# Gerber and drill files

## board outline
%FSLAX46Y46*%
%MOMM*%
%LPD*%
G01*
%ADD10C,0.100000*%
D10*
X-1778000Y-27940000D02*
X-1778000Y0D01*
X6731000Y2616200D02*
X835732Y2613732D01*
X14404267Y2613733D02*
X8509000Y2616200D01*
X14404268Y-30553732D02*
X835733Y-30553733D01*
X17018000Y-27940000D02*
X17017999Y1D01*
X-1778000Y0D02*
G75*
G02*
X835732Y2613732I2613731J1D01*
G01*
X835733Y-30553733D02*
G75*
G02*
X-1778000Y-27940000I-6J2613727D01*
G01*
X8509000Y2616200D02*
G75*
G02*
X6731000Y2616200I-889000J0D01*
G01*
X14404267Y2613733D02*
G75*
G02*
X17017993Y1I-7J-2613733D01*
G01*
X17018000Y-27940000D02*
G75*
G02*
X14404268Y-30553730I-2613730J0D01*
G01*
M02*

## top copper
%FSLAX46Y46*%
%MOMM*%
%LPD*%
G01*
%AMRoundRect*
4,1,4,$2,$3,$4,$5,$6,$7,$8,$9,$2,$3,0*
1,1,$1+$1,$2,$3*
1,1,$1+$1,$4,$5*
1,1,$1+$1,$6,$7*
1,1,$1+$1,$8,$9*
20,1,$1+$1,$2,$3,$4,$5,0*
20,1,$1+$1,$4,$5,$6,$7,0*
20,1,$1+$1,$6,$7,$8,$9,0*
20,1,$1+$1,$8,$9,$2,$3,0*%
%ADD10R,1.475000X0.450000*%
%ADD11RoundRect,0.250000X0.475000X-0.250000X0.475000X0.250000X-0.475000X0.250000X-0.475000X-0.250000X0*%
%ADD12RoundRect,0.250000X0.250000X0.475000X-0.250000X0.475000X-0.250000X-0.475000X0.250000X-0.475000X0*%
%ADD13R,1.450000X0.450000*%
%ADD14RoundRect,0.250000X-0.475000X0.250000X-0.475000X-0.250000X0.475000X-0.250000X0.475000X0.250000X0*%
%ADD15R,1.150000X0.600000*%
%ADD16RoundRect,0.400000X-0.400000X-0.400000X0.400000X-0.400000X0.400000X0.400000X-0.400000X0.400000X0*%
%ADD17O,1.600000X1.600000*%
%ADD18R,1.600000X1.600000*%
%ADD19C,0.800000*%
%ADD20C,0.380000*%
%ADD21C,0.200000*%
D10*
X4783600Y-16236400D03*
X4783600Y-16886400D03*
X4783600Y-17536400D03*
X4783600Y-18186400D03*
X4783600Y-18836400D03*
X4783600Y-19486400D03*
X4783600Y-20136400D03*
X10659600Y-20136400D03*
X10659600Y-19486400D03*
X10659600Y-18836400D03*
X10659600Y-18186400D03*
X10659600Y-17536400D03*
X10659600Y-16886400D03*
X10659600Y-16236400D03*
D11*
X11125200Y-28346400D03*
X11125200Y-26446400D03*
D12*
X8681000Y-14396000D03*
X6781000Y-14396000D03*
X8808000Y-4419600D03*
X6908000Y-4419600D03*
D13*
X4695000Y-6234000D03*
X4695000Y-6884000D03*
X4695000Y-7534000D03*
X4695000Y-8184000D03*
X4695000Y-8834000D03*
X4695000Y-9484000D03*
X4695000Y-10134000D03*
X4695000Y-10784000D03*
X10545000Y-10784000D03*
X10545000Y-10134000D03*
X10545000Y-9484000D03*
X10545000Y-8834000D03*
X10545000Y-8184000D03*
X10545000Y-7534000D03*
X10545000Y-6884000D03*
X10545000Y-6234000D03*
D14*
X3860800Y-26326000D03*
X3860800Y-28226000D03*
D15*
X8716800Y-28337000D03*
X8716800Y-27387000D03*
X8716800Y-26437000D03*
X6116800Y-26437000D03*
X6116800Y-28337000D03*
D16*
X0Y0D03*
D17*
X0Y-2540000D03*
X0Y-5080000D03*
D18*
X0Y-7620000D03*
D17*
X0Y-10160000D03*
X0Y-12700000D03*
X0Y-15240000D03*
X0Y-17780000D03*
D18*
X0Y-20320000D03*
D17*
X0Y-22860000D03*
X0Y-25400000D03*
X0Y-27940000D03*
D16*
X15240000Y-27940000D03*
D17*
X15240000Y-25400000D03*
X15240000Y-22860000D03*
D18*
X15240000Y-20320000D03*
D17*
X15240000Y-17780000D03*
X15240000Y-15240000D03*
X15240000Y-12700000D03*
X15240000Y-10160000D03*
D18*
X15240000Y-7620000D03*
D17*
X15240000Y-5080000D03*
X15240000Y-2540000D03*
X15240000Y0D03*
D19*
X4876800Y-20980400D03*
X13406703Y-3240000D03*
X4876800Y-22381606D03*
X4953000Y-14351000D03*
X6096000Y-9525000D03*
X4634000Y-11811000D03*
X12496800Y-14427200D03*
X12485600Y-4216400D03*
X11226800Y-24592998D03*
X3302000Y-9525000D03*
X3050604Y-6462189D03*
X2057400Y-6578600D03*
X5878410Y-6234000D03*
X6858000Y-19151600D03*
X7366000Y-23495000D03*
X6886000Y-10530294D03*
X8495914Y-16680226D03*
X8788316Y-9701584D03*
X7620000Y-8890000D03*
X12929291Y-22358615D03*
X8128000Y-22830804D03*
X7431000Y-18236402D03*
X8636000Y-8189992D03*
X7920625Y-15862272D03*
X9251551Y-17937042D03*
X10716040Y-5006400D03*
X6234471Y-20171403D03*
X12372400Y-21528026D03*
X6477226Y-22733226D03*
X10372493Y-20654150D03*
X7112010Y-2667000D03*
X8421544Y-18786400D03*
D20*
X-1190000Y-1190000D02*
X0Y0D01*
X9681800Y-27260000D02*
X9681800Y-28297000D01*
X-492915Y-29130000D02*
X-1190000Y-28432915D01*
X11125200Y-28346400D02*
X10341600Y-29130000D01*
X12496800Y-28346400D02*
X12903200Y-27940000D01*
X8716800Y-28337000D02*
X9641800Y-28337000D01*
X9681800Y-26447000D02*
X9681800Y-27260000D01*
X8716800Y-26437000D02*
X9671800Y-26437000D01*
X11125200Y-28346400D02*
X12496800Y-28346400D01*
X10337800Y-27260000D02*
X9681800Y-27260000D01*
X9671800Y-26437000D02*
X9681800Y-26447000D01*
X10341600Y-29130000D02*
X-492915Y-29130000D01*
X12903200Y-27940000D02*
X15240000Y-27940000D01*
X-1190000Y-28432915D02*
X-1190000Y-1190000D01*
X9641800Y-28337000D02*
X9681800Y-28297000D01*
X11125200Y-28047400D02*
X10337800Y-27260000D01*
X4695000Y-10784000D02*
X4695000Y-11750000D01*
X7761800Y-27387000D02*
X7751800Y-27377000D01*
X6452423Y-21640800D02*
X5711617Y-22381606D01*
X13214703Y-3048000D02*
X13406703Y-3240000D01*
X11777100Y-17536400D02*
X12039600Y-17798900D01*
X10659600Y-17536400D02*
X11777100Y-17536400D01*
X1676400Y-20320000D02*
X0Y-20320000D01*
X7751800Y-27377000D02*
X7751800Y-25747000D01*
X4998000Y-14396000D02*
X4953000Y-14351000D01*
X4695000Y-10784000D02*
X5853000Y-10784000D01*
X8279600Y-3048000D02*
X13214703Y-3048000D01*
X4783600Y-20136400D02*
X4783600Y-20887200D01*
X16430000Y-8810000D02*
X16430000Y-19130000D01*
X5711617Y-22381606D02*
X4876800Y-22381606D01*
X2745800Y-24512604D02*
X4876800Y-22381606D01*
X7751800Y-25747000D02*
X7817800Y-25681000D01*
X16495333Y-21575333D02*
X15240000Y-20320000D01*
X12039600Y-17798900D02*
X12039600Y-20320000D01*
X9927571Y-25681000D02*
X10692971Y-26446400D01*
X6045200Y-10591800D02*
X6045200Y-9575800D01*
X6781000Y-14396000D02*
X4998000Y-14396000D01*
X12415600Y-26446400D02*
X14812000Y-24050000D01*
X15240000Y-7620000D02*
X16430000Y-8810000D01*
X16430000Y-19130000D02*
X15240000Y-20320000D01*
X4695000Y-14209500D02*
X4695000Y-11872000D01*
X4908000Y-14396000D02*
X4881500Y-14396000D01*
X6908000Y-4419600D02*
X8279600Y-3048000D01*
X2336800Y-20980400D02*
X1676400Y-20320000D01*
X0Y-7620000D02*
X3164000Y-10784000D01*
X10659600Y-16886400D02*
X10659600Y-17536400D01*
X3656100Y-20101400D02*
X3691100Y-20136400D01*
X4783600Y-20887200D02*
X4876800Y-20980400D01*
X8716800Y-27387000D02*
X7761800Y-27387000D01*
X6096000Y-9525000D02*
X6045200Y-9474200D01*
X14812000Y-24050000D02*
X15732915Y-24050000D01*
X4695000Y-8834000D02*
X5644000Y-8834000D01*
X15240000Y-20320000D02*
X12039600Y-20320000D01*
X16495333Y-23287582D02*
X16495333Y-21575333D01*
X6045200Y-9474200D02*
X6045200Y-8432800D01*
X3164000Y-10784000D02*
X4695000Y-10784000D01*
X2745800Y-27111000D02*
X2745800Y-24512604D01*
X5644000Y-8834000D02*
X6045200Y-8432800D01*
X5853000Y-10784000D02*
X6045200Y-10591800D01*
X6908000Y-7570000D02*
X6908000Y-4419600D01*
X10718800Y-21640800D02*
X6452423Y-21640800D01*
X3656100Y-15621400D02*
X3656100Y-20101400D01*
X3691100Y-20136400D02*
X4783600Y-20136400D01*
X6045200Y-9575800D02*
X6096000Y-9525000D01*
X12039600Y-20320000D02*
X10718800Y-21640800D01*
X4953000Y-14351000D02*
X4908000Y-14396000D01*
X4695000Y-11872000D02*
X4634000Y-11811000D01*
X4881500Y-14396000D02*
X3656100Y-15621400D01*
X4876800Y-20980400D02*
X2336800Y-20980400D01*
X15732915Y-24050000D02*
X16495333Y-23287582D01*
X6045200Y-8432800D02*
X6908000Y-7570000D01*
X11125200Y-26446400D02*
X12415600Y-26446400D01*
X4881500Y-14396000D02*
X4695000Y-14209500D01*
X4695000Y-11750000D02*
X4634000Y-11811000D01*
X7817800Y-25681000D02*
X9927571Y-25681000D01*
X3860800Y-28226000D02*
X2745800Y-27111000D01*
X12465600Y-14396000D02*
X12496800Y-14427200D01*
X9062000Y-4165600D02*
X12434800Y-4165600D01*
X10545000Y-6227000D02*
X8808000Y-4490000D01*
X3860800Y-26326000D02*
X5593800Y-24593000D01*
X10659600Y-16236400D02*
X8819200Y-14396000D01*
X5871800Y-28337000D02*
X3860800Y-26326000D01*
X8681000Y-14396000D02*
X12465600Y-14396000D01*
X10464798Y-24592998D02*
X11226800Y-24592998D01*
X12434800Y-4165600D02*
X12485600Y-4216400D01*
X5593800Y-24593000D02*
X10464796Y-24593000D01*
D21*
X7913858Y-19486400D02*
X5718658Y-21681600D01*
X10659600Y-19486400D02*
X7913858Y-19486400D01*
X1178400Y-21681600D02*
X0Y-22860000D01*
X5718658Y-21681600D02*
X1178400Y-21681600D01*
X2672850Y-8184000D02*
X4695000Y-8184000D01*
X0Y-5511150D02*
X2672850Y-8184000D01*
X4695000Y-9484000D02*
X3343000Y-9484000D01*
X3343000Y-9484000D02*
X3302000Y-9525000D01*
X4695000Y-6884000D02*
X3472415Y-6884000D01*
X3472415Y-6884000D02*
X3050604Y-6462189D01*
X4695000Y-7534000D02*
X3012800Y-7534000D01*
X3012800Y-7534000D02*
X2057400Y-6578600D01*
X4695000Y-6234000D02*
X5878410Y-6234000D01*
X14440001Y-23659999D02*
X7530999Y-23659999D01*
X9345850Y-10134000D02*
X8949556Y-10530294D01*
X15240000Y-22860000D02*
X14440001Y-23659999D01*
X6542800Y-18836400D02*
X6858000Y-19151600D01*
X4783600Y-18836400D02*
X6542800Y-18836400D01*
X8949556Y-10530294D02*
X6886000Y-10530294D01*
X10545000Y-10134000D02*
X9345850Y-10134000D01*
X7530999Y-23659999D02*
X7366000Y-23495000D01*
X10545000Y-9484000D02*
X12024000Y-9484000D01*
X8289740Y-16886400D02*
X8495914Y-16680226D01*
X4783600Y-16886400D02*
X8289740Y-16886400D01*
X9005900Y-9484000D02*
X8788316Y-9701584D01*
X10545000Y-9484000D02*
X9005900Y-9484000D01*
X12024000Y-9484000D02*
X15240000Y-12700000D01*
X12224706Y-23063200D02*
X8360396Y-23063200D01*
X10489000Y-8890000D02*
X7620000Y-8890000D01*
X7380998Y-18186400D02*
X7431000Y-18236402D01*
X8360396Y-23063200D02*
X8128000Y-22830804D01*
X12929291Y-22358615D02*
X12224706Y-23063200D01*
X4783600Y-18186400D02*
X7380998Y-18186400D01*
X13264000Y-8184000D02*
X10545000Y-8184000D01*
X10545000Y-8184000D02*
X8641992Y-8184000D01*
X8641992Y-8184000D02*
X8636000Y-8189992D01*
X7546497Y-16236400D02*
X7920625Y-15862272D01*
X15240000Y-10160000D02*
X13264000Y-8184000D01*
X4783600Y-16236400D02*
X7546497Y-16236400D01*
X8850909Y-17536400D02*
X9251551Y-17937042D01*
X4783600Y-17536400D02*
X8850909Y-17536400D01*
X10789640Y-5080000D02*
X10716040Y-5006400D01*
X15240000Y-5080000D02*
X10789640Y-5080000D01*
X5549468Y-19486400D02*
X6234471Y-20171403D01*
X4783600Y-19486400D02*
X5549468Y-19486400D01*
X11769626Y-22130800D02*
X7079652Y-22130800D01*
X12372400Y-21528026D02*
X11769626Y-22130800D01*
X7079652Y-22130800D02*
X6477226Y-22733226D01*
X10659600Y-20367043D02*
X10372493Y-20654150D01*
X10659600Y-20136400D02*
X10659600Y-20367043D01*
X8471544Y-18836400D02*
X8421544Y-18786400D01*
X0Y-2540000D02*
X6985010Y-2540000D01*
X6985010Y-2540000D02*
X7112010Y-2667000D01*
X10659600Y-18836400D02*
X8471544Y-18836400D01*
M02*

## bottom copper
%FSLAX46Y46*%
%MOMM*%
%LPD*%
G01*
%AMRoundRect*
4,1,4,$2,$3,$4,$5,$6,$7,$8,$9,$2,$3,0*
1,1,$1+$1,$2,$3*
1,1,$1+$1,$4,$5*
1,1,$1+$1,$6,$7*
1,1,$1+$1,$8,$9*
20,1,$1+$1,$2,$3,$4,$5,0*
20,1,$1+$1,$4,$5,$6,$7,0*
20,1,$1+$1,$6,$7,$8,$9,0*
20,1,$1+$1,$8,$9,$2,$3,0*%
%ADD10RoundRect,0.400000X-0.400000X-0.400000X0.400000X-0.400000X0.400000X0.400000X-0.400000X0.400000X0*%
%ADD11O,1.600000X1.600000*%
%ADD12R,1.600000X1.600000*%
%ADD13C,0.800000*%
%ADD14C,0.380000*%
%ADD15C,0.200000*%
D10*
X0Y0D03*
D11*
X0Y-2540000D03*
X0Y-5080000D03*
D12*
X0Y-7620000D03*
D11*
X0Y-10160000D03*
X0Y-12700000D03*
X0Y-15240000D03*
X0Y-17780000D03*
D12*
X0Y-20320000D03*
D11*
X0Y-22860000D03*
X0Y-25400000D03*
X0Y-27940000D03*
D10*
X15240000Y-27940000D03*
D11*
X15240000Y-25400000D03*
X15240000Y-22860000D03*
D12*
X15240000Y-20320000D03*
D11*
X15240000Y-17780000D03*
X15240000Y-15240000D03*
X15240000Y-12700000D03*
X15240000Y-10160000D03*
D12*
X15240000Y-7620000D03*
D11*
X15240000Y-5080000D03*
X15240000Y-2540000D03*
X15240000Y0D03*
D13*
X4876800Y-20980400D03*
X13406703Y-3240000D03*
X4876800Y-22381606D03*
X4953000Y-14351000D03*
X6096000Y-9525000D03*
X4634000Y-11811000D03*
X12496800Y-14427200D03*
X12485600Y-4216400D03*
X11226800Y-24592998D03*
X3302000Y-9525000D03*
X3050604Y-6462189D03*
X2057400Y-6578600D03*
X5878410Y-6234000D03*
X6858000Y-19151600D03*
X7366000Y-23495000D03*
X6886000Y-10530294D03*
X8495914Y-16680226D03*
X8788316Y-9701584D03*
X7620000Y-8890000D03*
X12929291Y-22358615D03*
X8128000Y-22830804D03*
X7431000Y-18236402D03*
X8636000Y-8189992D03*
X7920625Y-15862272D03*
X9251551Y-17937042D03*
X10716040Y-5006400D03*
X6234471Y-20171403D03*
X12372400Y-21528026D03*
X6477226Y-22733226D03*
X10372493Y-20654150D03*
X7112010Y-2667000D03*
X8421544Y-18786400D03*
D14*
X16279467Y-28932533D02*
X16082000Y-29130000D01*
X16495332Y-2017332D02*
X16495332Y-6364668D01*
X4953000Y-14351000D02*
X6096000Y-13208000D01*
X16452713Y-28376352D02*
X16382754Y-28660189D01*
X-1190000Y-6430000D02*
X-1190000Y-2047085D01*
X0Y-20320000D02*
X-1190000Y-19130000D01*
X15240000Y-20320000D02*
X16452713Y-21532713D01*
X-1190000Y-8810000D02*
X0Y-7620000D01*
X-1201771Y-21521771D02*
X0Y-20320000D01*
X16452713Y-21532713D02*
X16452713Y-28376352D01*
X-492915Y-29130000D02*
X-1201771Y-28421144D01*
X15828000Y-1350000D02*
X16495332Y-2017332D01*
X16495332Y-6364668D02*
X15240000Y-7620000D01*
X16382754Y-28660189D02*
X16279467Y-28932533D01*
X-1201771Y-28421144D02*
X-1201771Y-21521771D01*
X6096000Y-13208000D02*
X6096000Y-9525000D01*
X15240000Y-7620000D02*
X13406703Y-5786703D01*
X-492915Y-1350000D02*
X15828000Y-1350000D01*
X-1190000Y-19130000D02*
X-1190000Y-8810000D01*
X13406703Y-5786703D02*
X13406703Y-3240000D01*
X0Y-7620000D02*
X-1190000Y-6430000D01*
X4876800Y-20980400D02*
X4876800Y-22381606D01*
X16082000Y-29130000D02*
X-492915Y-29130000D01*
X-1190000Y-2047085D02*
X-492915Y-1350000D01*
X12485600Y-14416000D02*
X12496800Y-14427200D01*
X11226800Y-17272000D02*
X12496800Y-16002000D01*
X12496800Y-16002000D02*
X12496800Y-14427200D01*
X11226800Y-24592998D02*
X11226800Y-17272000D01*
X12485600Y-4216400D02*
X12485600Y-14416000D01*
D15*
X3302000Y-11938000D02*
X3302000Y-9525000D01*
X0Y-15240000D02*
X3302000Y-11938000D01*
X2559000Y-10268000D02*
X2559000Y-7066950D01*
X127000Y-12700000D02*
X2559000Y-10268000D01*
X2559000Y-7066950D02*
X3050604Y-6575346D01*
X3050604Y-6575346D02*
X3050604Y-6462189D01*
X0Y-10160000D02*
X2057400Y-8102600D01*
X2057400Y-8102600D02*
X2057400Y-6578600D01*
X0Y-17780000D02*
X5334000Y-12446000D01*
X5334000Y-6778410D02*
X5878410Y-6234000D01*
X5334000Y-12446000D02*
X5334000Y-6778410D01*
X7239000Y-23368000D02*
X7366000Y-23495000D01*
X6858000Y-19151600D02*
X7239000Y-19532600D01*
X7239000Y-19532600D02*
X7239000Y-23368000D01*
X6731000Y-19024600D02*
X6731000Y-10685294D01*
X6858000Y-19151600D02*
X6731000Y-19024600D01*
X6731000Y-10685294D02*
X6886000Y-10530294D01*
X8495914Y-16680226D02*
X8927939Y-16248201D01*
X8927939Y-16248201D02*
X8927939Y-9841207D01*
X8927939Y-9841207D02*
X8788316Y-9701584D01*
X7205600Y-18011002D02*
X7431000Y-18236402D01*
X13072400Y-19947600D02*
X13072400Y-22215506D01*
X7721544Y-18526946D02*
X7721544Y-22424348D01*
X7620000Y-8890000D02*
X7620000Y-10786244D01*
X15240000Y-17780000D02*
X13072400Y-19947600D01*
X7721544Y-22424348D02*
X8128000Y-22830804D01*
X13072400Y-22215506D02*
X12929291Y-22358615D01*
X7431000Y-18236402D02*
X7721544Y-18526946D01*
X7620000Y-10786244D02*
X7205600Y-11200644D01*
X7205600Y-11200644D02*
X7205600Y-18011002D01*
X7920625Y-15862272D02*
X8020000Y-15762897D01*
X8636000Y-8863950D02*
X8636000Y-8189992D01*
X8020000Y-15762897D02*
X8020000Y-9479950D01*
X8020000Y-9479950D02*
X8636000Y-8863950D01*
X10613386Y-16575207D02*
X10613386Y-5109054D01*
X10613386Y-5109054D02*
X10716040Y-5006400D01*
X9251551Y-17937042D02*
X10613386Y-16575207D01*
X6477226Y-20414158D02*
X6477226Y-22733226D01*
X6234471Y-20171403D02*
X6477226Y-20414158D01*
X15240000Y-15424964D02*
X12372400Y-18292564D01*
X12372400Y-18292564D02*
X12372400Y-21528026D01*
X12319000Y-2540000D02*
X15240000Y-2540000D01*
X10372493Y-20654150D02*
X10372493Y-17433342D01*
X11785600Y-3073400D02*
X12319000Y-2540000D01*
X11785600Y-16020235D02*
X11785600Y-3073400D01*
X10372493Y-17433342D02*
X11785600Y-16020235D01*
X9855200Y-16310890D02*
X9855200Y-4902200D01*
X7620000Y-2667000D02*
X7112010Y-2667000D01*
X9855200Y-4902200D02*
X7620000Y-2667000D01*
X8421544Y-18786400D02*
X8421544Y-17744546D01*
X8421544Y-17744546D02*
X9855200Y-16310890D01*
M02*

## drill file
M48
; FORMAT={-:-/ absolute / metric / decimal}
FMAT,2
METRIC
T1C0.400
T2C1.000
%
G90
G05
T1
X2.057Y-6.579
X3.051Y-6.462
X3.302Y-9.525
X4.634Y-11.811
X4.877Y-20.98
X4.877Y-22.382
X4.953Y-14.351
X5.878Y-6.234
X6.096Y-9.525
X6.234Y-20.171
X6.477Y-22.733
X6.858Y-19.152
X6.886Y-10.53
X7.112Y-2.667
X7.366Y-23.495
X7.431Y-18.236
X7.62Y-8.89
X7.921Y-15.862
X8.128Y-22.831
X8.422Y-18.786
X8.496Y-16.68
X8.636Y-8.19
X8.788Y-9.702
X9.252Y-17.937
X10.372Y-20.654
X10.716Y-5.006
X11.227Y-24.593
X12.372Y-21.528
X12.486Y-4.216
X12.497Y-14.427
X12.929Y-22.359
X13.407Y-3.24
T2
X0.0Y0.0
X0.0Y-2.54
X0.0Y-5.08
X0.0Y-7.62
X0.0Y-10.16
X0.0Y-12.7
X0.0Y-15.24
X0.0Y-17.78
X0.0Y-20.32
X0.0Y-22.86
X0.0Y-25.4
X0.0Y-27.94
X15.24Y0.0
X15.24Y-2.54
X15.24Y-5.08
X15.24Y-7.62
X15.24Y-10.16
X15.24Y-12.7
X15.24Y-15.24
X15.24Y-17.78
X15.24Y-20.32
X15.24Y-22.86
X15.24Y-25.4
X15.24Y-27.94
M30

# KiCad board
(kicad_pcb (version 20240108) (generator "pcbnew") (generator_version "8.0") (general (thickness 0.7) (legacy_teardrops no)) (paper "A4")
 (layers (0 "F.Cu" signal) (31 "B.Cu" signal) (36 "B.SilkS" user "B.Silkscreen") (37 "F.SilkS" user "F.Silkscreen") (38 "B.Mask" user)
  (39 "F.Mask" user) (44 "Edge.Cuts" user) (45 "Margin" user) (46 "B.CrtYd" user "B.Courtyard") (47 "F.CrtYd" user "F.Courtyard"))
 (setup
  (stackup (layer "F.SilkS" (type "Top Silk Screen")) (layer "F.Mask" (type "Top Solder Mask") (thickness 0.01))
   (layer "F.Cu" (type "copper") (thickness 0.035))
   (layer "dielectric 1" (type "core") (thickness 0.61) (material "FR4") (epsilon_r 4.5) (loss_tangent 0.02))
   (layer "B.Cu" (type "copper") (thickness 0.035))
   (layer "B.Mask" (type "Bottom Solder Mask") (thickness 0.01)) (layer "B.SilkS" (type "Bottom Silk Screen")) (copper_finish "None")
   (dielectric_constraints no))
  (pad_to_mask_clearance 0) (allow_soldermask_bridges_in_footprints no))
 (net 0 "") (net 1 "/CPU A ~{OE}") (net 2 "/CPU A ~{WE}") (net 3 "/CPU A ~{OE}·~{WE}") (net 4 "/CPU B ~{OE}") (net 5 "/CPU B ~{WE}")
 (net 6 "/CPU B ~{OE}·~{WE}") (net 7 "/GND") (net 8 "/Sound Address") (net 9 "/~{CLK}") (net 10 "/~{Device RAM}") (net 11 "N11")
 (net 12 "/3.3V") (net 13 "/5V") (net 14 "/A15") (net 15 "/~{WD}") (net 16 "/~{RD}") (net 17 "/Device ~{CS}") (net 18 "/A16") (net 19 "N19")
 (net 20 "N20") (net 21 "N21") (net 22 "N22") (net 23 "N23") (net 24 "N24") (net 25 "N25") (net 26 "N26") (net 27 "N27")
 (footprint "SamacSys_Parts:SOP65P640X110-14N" (layer "F.Cu") (at 7.7216 18.1864)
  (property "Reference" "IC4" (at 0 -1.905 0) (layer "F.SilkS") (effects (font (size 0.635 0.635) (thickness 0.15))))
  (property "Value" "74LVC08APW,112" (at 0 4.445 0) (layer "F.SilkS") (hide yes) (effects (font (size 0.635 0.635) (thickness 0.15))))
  (pad "1" smd rect (at -2.938 -1.95 90) (size 0.45 1.475) (layers "F.Cu" "F.Paste" "F.Mask") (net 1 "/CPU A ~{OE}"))
  (pad "2" smd rect (at -2.938 -1.3 90) (size 0.45 1.475) (layers "F.Cu" "F.Paste" "F.Mask") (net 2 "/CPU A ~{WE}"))
  (pad "3" smd rect (at -2.938 -0.65 90) (size 0.45 1.475) (layers "F.Cu" "F.Paste" "F.Mask") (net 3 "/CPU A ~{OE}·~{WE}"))
  (pad "4" smd rect (at -2.938 0 90) (size 0.45 1.475) (layers "F.Cu" "F.Paste" "F.Mask") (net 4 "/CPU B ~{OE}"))
  (pad "5" smd rect (at -2.938 0.65 90) (size 0.45 1.475) (layers "F.Cu" "F.Paste" "F.Mask") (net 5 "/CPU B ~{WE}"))
  (pad "6" smd rect (at -2.938 1.3 90) (size 0.45 1.475) (layers "F.Cu" "F.Paste" "F.Mask") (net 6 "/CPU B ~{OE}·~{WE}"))
  (pad "7" smd rect (at -2.938 1.95 90) (size 0.45 1.475) (layers "F.Cu" "F.Paste" "F.Mask") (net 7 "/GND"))
  (pad "8" smd rect (at 2.938 1.95 90) (size 0.45 1.475) (layers "F.Cu" "F.Paste" "F.Mask") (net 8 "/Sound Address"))
  (pad "9" smd rect (at 2.938 1.3 90) (size 0.45 1.475) (layers "F.Cu" "F.Paste" "F.Mask") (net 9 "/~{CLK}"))
  (pad "10" smd rect (at 2.938 0.65 90) (size 0.45 1.475) (layers "F.Cu" "F.Paste" "F.Mask") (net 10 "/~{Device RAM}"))
  (pad "11" smd rect (at 2.938 0 90) (size 0.45 1.475) (layers "F.Cu" "F.Paste" "F.Mask") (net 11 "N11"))
  (pad "12" smd rect (at 2.938 -0.65 90) (size 0.45 1.475) (layers "F.Cu" "F.Paste" "F.Mask") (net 7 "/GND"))
  (pad "13" smd rect (at 2.938 -1.3 90) (size 0.45 1.475) (layers "F.Cu" "F.Paste" "F.Mask") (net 7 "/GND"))
  (pad "14" smd rect (at 2.938 -1.95 90) (size 0.45 1.475) (layers "F.Cu" "F.Paste" "F.Mask") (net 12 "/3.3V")))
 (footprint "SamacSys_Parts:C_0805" (layer "F.Cu") (at 11.1252 27.4124)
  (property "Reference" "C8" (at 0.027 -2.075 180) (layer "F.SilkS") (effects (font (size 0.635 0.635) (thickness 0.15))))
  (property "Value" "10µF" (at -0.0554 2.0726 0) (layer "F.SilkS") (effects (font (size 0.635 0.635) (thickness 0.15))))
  (pad "1" smd roundrect (at 0 0.934 90) (size 1 1.45) (layers "F.Cu" "F.Paste" "F.Mask") (roundrect_rratio 0.25) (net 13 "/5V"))
  (pad "2" smd roundrect (at 0 -0.966 90) (size 1 1.45) (layers "F.Cu" "F.Paste" "F.Mask") (roundrect_rratio 0.25) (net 7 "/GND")))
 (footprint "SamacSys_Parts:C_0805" (layer "F.Cu") (at 7.747 14.396 90)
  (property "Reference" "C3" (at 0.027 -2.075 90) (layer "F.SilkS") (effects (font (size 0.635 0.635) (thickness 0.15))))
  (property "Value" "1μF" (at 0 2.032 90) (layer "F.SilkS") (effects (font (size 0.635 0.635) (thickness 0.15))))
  (pad "1" smd roundrect (at 0 0.934 180) (size 1 1.45) (layers "F.Cu" "F.Paste" "F.Mask") (roundrect_rratio 0.25) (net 12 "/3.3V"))
  (pad "2" smd roundrect (at 0 -0.966 180) (size 1 1.45) (layers "F.Cu" "F.Paste" "F.Mask") (roundrect_rratio 0.25) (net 7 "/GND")))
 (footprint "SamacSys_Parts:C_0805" (layer "F.Cu") (at 7.874 4.4196 90)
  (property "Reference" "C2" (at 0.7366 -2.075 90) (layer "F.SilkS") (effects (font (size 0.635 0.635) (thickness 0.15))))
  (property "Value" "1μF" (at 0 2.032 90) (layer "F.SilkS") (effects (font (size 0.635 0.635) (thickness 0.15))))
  (pad "1" smd roundrect (at 0 0.934 180) (size 1 1.45) (layers "F.Cu" "F.Paste" "F.Mask") (roundrect_rratio 0.25) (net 12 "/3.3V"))
  (pad "2" smd roundrect (at 0 -0.966 180) (size 1 1.45) (layers "F.Cu" "F.Paste" "F.Mask") (roundrect_rratio 0.25) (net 7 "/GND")))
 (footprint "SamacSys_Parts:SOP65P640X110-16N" (layer "F.Cu") (at 7.62 8.509)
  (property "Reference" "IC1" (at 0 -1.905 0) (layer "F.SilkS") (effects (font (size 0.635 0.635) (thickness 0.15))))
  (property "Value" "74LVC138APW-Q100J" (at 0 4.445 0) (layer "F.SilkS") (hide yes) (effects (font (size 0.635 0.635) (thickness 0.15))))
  (pad "1" smd rect (at -2.925 -2.275 90) (size 0.45 1.45) (layers "F.Cu" "F.Paste" "F.Mask") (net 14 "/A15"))
  (pad "2" smd rect (at -2.925 -1.625 90) (size 0.45 1.45) (layers "F.Cu" "F.Paste" "F.Mask") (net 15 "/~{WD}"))
  (pad "3" smd rect (at -2.925 -0.975 90) (size 0.45 1.45) (layers "F.Cu" "F.Paste" "F.Mask") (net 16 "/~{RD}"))
  (pad "4" smd rect (at -2.925 -0.325 90) (size 0.45 1.45) (layers "F.Cu" "F.Paste" "F.Mask") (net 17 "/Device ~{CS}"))
  (pad "5" smd rect (at -2.925 0.325 90) (size 0.45 1.45) (layers "F.Cu" "F.Paste" "F.Mask") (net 7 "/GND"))
  (pad "6" smd rect (at -2.925 0.975 90) (size 0.45 1.45) (layers "F.Cu" "F.Paste" "F.Mask") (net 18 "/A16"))
  (pad "7" smd rect (at -2.925 1.625 90) (size 0.45 1.45) (layers "F.Cu" "F.Paste" "F.Mask") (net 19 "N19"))
  (pad "8" smd rect (at -2.925 2.275 90) (size 0.45 1.45) (layers "F.Cu" "F.Paste" "F.Mask") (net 7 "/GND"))
  (pad "9" smd rect (at 2.925 2.275 90) (size 0.45 1.45) (layers "F.Cu" "F.Paste" "F.Mask") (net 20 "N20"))
  (pad "10" smd rect (at 2.925 1.625 90) (size 0.45 1.45) (layers "F.Cu" "F.Paste" "F.Mask") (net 5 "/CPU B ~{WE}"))
  (pad "11" smd rect (at 2.925 0.975 90) (size 0.45 1.45) (layers "F.Cu" "F.Paste" "F.Mask") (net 2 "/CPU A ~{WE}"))
  (pad "12" smd rect (at 2.925 0.325 90) (size 0.45 1.45) (layers "F.Cu" "F.Paste" "F.Mask") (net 4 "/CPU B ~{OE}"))
  (pad "13" smd rect (at 2.925 -0.325 90) (size 0.45 1.45) (layers "F.Cu" "F.Paste" "F.Mask") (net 1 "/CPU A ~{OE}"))
  (pad "14" smd rect (at 2.925 -0.975 90) (size 0.45 1.45) (layers "F.Cu" "F.Paste" "F.Mask") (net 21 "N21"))
  (pad "15" smd rect (at 2.925 -1.625 90) (size 0.45 1.45) (layers "F.Cu" "F.Paste" "F.Mask") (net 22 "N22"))
  (pad "16" smd rect (at 2.925 -2.275 90) (size 0.45 1.45) (layers "F.Cu" "F.Paste" "F.Mask") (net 12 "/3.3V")))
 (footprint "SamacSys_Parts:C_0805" (layer "F.Cu") (at 3.8608 27.26 180)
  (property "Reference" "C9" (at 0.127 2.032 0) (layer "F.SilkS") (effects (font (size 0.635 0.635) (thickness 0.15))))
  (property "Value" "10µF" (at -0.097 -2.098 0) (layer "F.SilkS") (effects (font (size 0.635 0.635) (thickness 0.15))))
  (pad "1" smd roundrect (at 0 0.934 270) (size 1 1.45) (layers "F.Cu" "F.Paste" "F.Mask") (roundrect_rratio 0.25) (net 12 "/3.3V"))
  (pad "2" smd roundrect (at 0 -0.966 270) (size 1 1.45) (layers "F.Cu" "F.Paste" "F.Mask") (roundrect_rratio 0.25) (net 7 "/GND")))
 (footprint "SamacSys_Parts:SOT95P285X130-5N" (layer "F.Cu") (at 7.4168 27.387 180)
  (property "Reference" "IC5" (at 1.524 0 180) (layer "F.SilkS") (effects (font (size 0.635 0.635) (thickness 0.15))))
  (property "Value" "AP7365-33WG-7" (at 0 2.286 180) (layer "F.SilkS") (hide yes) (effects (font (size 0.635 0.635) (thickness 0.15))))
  (pad "1" smd rect (at -1.3 -0.95 270) (size 0.6 1.15) (layers "F.Cu" "F.Paste" "F.Mask") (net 13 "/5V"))
  (pad "2" smd rect (at -1.3 0 270) (size 0.6 1.15) (layers "F.Cu" "F.Paste" "F.Mask") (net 7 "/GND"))
  (pad "3" smd rect (at -1.3 0.95 270) (size 0.6 1.15) (layers "F.Cu" "F.Paste" "F.Mask") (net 13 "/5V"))
  (pad "4" smd rect (at 1.3 0.95 270) (size 0.6 1.15) (layers "F.Cu" "F.Paste" "F.Mask") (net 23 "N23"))
  (pad "5" smd rect (at 1.3 -0.95 270) (size 0.6 1.15) (layers "F.Cu" "F.Paste" "F.Mask") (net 12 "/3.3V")))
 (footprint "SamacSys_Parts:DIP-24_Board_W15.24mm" (layer "F.Cu") (at 0 0)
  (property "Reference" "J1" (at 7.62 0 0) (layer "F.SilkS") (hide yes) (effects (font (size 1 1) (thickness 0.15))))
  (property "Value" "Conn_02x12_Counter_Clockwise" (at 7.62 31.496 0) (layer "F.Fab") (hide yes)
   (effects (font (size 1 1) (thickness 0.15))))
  (fp_line (start -1.778 27.94) (end -1.778 0) (stroke (width 0.1) (type solid)) (layer "Edge.Cuts"))
  (fp_line (start 6.731 -2.6162) (end 0.835732 -2.613732) (stroke (width 0.1) (type solid)) (layer "Edge.Cuts"))
  (fp_line (start 14.404267 -2.613733) (end 8.509 -2.6162) (stroke (width 0.1) (type solid)) (layer "Edge.Cuts"))
  (fp_line (start 14.404268 30.553732) (end 0.835733 30.553733) (stroke (width 0.1) (type solid)) (layer "Edge.Cuts"))
  (fp_line (start 17.018 27.94) (end 17.017999 -0.000001) (stroke (width 0.1) (type solid)) (layer "Edge.Cuts"))
  (fp_arc (start -1.778 0) (mid -1.012456 -1.848188) (end 0.835732 -2.613732) (stroke (width 0.1) (type solid)) (layer "Edge.Cuts"))
  (fp_arc (start 0.835733 30.553733) (mid -1.012457 29.78819) (end -1.778 27.94) (stroke (width 0.1) (type solid)) (layer "Edge.Cuts"))
  (fp_arc (start 8.509 -2.6162) (mid 7.62 -1.7272) (end 6.731 -2.6162) (stroke (width 0.1) (type default)) (layer "Edge.Cuts"))
  (fp_arc (start 14.404267 -2.613733) (mid 16.252453 -1.848189) (end 17.017999 -0.000001) (stroke (width 0.1) (type solid))
   (layer "Edge.Cuts"))
  (fp_arc (start 17.018 27.94) (mid 16.252456 29.788187) (end 14.404268 30.553732) (stroke (width 0.1) (type solid)) (layer "Edge.Cuts"))
  (pad "1" thru_hole roundrect (at 0 0) (size 1.6 1.6) (drill 1) (layers "*.Cu" "*.Mask") (remove_unused_layers no) (roundrect_rratio 0.25)
   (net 13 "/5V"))
  (pad "2" thru_hole oval (at 0 2.54) (size 1.6 1.6) (drill 1) (layers "*.Cu" "*.Mask") (remove_unused_layers no) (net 10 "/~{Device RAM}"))
  (pad "3" thru_hole oval (at 0 5.08) (size 1.6 1.6) (drill 1) (layers "*.Cu" "*.Mask") (remove_unused_layers no) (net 17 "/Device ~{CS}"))
  (pad "4" thru_hole rect (at 0 7.62) (size 1.6 1.6) (drill 1) (layers "*.Cu" "*.Mask") (remove_unused_layers no) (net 7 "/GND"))
  (pad "5" thru_hole oval (at 0 10.16) (size 1.6 1.6) (drill 1) (layers "*.Cu" "*.Mask") (remove_unused_layers no) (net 16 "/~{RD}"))
  (pad "6" thru_hole oval (at 0 12.7) (size 1.6 1.6) (drill 1) (layers "*.Cu" "*.Mask") (remove_unused_layers no) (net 15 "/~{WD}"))
  (pad "7" thru_hole oval (at 0 15.24) (size 1.6 1.6) (drill 1) (layers "*.Cu" "*.Mask") (remove_unused_layers no) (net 18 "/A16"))
  (pad "8" thru_hole oval (at 0 17.78) (size 1.6 1.6) (drill 1) (layers "*.Cu" "*.Mask") (remove_unused_layers no) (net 14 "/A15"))
  (pad "9" thru_hole rect (at 0 20.32) (size 1.6 1.6) (drill 1) (layers "*.Cu" "*.Mask") (remove_unused_layers no) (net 7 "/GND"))
  (pad "10" thru_hole oval (at 0 22.86) (size 1.6 1.6) (drill 1) (layers "*.Cu" "*.Mask") (remove_unused_layers no) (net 9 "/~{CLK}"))
  (pad "11" thru_hole oval (at 0 25.4) (size 1.6 1.6) (drill 1) (layers "*.Cu" "*.Mask") (remove_unused_layers no) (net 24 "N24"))
  (pad "12" thru_hole oval (at 0 27.94) (size 1.6 1.6) (drill 1) (layers "*.Cu" "*.Mask") (remove_unused_layers no) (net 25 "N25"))
  (pad "13" thru_hole roundrect (at 15.24 27.94) (size 1.6 1.6) (drill 1) (layers "*.Cu" "*.Mask") (remove_unused_layers no)
   (roundrect_rratio 0.25) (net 13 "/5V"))
  (pad "14" thru_hole oval (at 15.24 25.4) (size 1.6 1.6) (drill 1) (layers "*.Cu" "*.Mask") (remove_unused_layers no) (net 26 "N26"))
  (pad "15" thru_hole oval (at 15.24 22.86) (size 1.6 1.6) (drill 1) (layers "*.Cu" "*.Mask") (remove_unused_layers no)
   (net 5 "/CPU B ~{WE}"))
  (pad "16" thru_hole rect (at 15.24 20.32) (size 1.6 1.6) (drill 1) (layers "*.Cu" "*.Mask") (remove_unused_layers no) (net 7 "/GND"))
  (pad "17" thru_hole oval (at 15.24 17.78 180) (size 1.6 1.6) (drill 1) (layers "*.Cu" "*.Mask") (remove_unused_layers no)
   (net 4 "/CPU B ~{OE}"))
  (pad "18" thru_hole oval (at 15.24 15.24 180) (size 1.6 1.6) (drill 1) (layers "*.Cu" "*.Mask") (remove_unused_layers no)
   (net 6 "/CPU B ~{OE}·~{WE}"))
  (pad "19" thru_hole oval (at 15.24 12.7 180) (size 1.6 1.6) (drill 1) (layers "*.Cu" "*.Mask") (remove_unused_layers no)
   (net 2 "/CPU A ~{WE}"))
  (pad "20" thru_hole oval (at 15.24 10.16 180) (size 1.6 1.6) (drill 1) (layers "*.Cu" "*.Mask") (remove_unused_layers no)
   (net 1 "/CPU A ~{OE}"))
  (pad "21" thru_hole rect (at 15.24 7.62) (size 1.6 1.6) (drill 1) (layers "*.Cu" "*.Mask") (remove_unused_layers no) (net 7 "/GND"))
  (pad "22" thru_hole oval (at 15.24 5.08) (size 1.6 1.6) (drill 1) (layers "*.Cu" "*.Mask") (remove_unused_layers no)
   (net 3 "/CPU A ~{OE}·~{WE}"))
  (pad "23" thru_hole oval (at 15.24 2.54) (size 1.6 1.6) (drill 1) (layers "*.Cu" "*.Mask") (remove_unused_layers no)
   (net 8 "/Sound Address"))
  (pad "24" thru_hole oval (at 15.24 0) (size 1.6 1.6) (drill 1) (layers "*.Cu" "*.Mask") (remove_unused_layers no) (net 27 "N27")))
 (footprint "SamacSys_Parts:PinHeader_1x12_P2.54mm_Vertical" (layer "B.Cu") (at 0 0 180)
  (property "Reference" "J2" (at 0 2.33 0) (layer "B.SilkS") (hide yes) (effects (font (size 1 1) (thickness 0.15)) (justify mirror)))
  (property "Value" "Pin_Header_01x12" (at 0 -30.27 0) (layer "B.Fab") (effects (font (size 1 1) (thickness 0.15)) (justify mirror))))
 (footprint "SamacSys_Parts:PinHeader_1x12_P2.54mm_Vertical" (layer "B.Cu") (at 15.24 0 180)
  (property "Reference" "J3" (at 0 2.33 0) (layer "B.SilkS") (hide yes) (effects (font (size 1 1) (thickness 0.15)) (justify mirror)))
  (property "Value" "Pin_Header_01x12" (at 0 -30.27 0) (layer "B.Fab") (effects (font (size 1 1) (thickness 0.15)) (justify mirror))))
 (segment (start -1.19 1.19) (end 0 0) (width 0.38) (layer "F.Cu") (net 13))
 (segment (start 9.6818 27.26) (end 9.6818 28.297) (width 0.38) (layer "F.Cu") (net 13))
 (segment (start -0.492915 29.13) (end -1.19 28.432915) (width 0.38) (layer "F.Cu") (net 13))
 (segment (start 11.1252 28.3464) (end 10.3416 29.13) (width 0.38) (layer "F.Cu") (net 13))
 (segment (start 12.4968 28.3464) (end 12.9032 27.94) (width 0.38) (layer "F.Cu") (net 13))
 (segment (start 8.7168 28.337) (end 9.6418 28.337) (width 0.38) (layer "F.Cu") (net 13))
 (segment (start 9.6818 26.447) (end 9.6818 27.26) (width 0.38) (layer "F.Cu") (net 13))
 (segment (start 8.7168 26.437) (end 9.6718 26.437) (width 0.38) (layer "F.Cu") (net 13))
 (segment (start 11.1252 28.3464) (end 12.4968 28.3464) (width 0.38) (layer "F.Cu") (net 13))
 (segment (start 10.3378 27.26) (end 9.6818 27.26) (width 0.38) (layer "F.Cu") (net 13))
 (segment (start 9.6718 26.437) (end 9.6818 26.447) (width 0.38) (layer "F.Cu") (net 13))
 (segment (start 10.3416 29.13) (end -0.492915 29.13) (width 0.38) (layer "F.Cu") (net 13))
 (segment (start 12.9032 27.94) (end 15.24 27.94) (width 0.38) (layer "F.Cu") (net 13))
 (segment (start -1.19 28.432915) (end -1.19 1.19) (width 0.38) (layer "F.Cu") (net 13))
 (segment (start 9.6418 28.337) (end 9.6818 28.297) (width 0.38) (layer "F.Cu") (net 13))
 (segment (start 11.1252 28.0474) (end 10.3378 27.26) (width 0.38) (layer "F.Cu") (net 13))
 (segment (start 4.695 10.784) (end 4.695 11.75) (width 0.38) (layer "F.Cu") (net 7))
 (segment (start 7.7618 27.387) (end 7.7518 27.377) (width 0.38) (layer "F.Cu") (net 7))
 (segment (start 6.452423 21.6408) (end 5.711617 22.381606) (width 0.38) (layer "F.Cu") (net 7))
 (segment (start 13.214703 3.048) (end 13.406703 3.24) (width 0.38) (layer "F.Cu") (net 7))
 (segment (start 11.7771 17.5364) (end 12.0396 17.7989) (width 0.38) (layer "F.Cu") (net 7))
 (segment (start 10.6596 17.5364) (end 11.7771 17.5364) (width 0.38) (layer "F.Cu") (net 7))
 (segment (start 1.6764 20.32) (end 0 20.32) (width 0.38) (layer "F.Cu") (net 7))
 (segment (start 7.7518 27.377) (end 7.7518 25.747) (width 0.38) (layer "F.Cu") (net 7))
 (segment (start 4.998 14.396) (end 4.953 14.351) (width 0.38) (layer "F.Cu") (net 7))
 (segment (start 4.695 10.784) (end 5.853 10.784) (width 0.38) (layer "F.Cu") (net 7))
 (segment (start 8.2796 3.048) (end 13.214703 3.048) (width 0.38) (layer "F.Cu") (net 7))
 (segment (start 4.7836 20.1364) (end 4.7836 20.8872) (width 0.38) (layer "F.Cu") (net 7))
 (segment (start 16.43 8.81) (end 16.43 19.13) (width 0.38) (layer "F.Cu") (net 7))
 (segment (start 5.711617 22.381606) (end 4.8768 22.381606) (width 0.38) (layer "F.Cu") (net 7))
 (segment (start 2.7458 24.512604) (end 4.8768 22.381606) (width 0.38) (layer "F.Cu") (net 7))
 (segment (start 7.7518 25.747) (end 7.8178 25.681) (width 0.38) (layer "F.Cu") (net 7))
 (segment (start 16.495333 21.575333) (end 15.24 20.32) (width 0.38) (layer "F.Cu") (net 7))
 (segment (start 12.0396 17.7989) (end 12.0396 20.32) (width 0.38) (layer "F.Cu") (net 7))
 (segment (start 9.927571 25.681) (end 10.692971 26.4464) (width 0.38) (layer "F.Cu") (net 7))
 (segment (start 6.0452 10.5918) (end 6.0452 9.5758) (width 0.38) (layer "F.Cu") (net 7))
 (segment (start 6.781 14.396) (end 4.998 14.396) (width 0.38) (layer "F.Cu") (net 7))
 (segment (start 12.4156 26.4464) (end 14.812 24.05) (width 0.38) (layer "F.Cu") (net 7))
 (segment (start 15.24 7.62) (end 16.43 8.81) (width 0.38) (layer "F.Cu") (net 7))
 (segment (start 16.43 19.13) (end 15.24 20.32) (width 0.38) (layer "F.Cu") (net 7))
 (segment (start 4.695 14.2095) (end 4.695 11.872) (width 0.38) (layer "F.Cu") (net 7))
 (segment (start 4.908 14.396) (end 4.8815 14.396) (width 0.38) (layer "F.Cu") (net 7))
 (segment (start 6.908 4.4196) (end 8.2796 3.048) (width 0.38) (layer "F.Cu") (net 7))
 (segment (start 2.3368 20.9804) (end 1.6764 20.32) (width 0.38) (layer "F.Cu") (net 7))
 (segment (start 0 7.62) (end 3.164 10.784) (width 0.38) (layer "F.Cu") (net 7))
 (segment (start 10.6596 16.8864) (end 10.6596 17.5364) (width 0.38) (layer "F.Cu") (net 7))
 (segment (start 3.6561 20.1014) (end 3.6911 20.1364) (width 0.38) (layer "F.Cu") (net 7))
 (segment (start 4.7836 20.8872) (end 4.8768 20.9804) (width 0.38) (layer "F.Cu") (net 7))
 (segment (start 8.7168 27.387) (end 7.7618 27.387) (width 0.38) (layer "F.Cu") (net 7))
 (segment (start 6.096 9.525) (end 6.0452 9.4742) (width 0.38) (layer "F.Cu") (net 7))
 (segment (start 14.812 24.05) (end 15.732915 24.05) (width 0.38) (layer "F.Cu") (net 7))
 (segment (start 4.695 8.834) (end 5.644 8.834) (width 0.38) (layer "F.Cu") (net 7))
 (segment (start 15.24 20.32) (end 12.0396 20.32) (width 0.38) (layer "F.Cu") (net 7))
 (segment (start 16.495333 23.287582) (end 16.495333 21.575333) (width 0.38) (layer "F.Cu") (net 7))
 (segment (start 6.0452 9.4742) (end 6.0452 8.4328) (width 0.38) (layer "F.Cu") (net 7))
 (segment (start 3.164 10.784) (end 4.695 10.784) (width 0.38) (layer "F.Cu") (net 7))
 (segment (start 2.7458 27.111) (end 2.7458 24.512604) (width 0.38) (layer "F.Cu") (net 7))
 (segment (start 5.644 8.834) (end 6.0452 8.4328) (width 0.38) (layer "F.Cu") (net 7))
 (segment (start 5.853 10.784) (end 6.0452 10.5918) (width 0.38) (layer "F.Cu") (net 7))
 (segment (start 6.908 7.57) (end 6.908 4.4196) (width 0.38) (layer "F.Cu") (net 7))
 (segment (start 10.7188 21.6408) (end 6.452423 21.6408) (width 0.38) (layer "F.Cu") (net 7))
 (segment (start 3.6561 15.6214) (end 3.6561 20.1014) (width 0.38) (layer "F.Cu") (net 7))
 (segment (start 3.6911 20.1364) (end 4.7836 20.1364) (width 0.38) (layer "F.Cu") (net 7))
 (segment (start 6.0452 9.5758) (end 6.096 9.525) (width 0.38) (layer "F.Cu") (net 7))
 (segment (start 12.0396 20.32) (end 10.7188 21.6408) (width 0.38) (layer "F.Cu") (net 7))
 (segment (start 4.953 14.351) (end 4.908 14.396) (width 0.38) (layer "F.Cu") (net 7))
 (segment (start 4.695 11.872) (end 4.634 11.811) (width 0.38) (layer "F.Cu") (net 7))
 (segment (start 4.8815 14.396) (end 3.6561 15.6214) (width 0.38) (layer "F.Cu") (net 7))
 (segment (start 4.8768 20.9804) (end 2.3368 20.9804) (width 0.38) (layer "F.Cu") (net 7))
 (segment (start 15.732915 24.05) (end 16.495333 23.287582) (width 0.38) (layer "F.Cu") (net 7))
 (segment (start 6.0452 8.4328) (end 6.908 7.57) (width 0.38) (layer "F.Cu") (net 7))
 (segment (start 11.1252 26.4464) (end 12.4156 26.4464) (width 0.38) (layer "F.Cu") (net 7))
 (segment (start 4.8815 14.396) (end 4.695 14.2095) (width 0.38) (layer "F.Cu") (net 7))
 (segment (start 4.695 11.75) (end 4.634 11.811) (width 0.38) (layer "F.Cu") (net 7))
 (segment (start 7.8178 25.681) (end 9.927571 25.681) (width 0.38) (layer "F.Cu") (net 7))
 (segment (start 3.8608 28.226) (end 2.7458 27.111) (width 0.38) (layer "F.Cu") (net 7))
 (via (at 4.8768 20.9804) (size 0.8) (drill 0.4) (layers "F.Cu" "B.Cu") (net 7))
 (via (at 13.406703 3.24) (size 0.8) (drill 0.4) (layers "F.Cu" "B.Cu") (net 7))
 (via (at 4.8768 22.381606) (size 0.8) (drill 0.4) (layers "F.Cu" "B.Cu") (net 7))
 (via (at 4.953 14.351) (size 0.8) (drill 0.4) (layers "F.Cu" "B.Cu") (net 7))
 (via (at 6.096 9.525) (size 0.8) (drill 0.4) (layers "F.Cu" "B.Cu") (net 7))
 (via (at 4.634 11.811) (size 0.8) (drill 0.4) (layers "F.Cu" "B.Cu") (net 7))
 (segment (start 16.279467 28.932533) (end 16.082 29.13) (width 0.38) (layer "B.Cu") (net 7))
 (segment (start 16.495332 2.017332) (end 16.495332 6.364668) (width 0.38) (layer "B.Cu") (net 7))
 (segment (start 4.953 14.351) (end 6.096 13.208) (width 0.38) (layer "B.Cu") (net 7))
 (segment (start 16.452713 28.376352) (end 16.382754 28.660189) (width 0.38) (layer "B.Cu") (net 7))
 (segment (start -1.19 6.43) (end -1.19 2.047085) (width 0.38) (layer "B.Cu") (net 7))
 (segment (start 0 20.32) (end -1.19 19.13) (width 0.38) (layer "B.Cu") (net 7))
 (segment (start 15.24 20.32) (end 16.452713 21.532713) (width 0.38) (layer "B.Cu") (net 7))
 (segment (start -1.19 8.81) (end 0 7.62) (width 0.38) (layer "B.Cu") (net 7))
 (segment (start -1.201771 21.521771) (end 0 20.32) (width 0.38) (layer "B.Cu") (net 7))
 (segment (start 16.452713 21.532713) (end 16.452713 28.376352) (width 0.38) (layer "B.Cu") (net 7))
 (segment (start -0.492915 29.13) (end -1.201771 28.421144) (width 0.38) (layer "B.Cu") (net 7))
 (segment (start 15.828 1.35) (end 16.495332 2.017332) (width 0.38) (layer "B.Cu") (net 7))
 (segment (start 16.495332 6.364668) (end 15.24 7.62) (width 0.38) (layer "B.Cu") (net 7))
 (segment (start 16.382754 28.660189) (end 16.279467 28.932533) (width 0.38) (layer "B.Cu") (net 7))
 (segment (start -1.201771 28.421144) (end -1.201771 21.521771) (width 0.38) (layer "B.Cu") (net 7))
 (segment (start 6.096 13.208) (end 6.096 9.525) (width 0.38) (layer "B.Cu") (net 7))
 (segment (start 15.24 7.62) (end 13.406703 5.786703) (width 0.38) (layer "B.Cu") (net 7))
 (segment (start -0.492915 1.35) (end 15.828 1.35) (width 0.38) (layer "B.Cu") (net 7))
 (segment (start -1.19 19.13) (end -1.19 8.81) (width 0.38) (layer "B.Cu") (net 7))
 (segment (start 13.406703 5.786703) (end 13.406703 3.24) (width 0.38) (layer "B.Cu") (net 7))
 (segment (start 0 7.62) (end -1.19 6.43) (width 0.38) (layer "B.Cu") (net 7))
 (segment (start 4.8768 20.9804) (end 4.8768 22.381606) (width 0.38) (layer "B.Cu") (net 7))
 (segment (start 16.082 29.13) (end -0.492915 29.13) (width 0.38) (layer "B.Cu") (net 7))
 (segment (start -1.19 2.047085) (end -0.492915 1.35) (width 0.38) (layer "B.Cu") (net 7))
 (segment (start 12.4656 14.396) (end 12.4968 14.4272) (width 0.38) (layer "F.Cu") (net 12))
 (segment (start 9.062 4.1656) (end 12.4348 4.1656) (width 0.38) (layer "F.Cu") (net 12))
 (segment (start 10.545 6.227) (end 8.808 4.49) (width 0.38) (layer "F.Cu") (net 12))
 (segment (start 3.8608 26.326) (end 5.5938 24.593) (width 0.38) (layer "F.Cu") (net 12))
 (segment (start 10.6596 16.2364) (end 8.8192 14.396) (width 0.38) (layer "F.Cu") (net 12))
 (segment (start 5.8718 28.337) (end 3.8608 26.326) (width 0.38) (layer "F.Cu") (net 12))
 (segment (start 8.681 14.396) (end 12.4656 14.396) (width 0.38) (layer "F.Cu") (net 12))
 (segment (start 10.464798 24.592998) (end 11.2268 24.592998) (width 0.38) (layer "F.Cu") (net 12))
 (segment (start 12.4348 4.1656) (end 12.4856 4.2164) (width 0.38) (layer "F.Cu") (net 12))
 (segment (start 5.5938 24.593) (end 10.464796 24.593) (width 0.38) (layer "F.Cu") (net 12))
 (via (at 12.4968 14.4272) (size 0.8) (drill 0.4) (layers "F.Cu" "B.Cu") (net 12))
 (via (at 12.4856 4.2164) (size 0.8) (drill 0.4) (layers "F.Cu" "B.Cu") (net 12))
 (via (at 11.2268 24.592998) (size 0.8) (drill 0.4) (layers "F.Cu" "B.Cu") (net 12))
 (segment (start 12.4856 14.416) (end 12.4968 14.4272) (width 0.38) (layer "B.Cu") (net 12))
 (segment (start 11.2268 17.272) (end 12.4968 16.002) (width 0.38) (layer "B.Cu") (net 12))
 (segment (start 12.4968 16.002) (end 12.4968 14.4272) (width 0.38) (layer "B.Cu") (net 12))
 (segment (start 11.2268 24.592998) (end 11.2268 17.272) (width 0.38) (layer "B.Cu") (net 12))
 (segment (start 12.4856 4.2164) (end 12.4856 14.416) (width 0.38) (layer "B.Cu") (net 12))
 (segment (start 7.913858 19.4864) (end 5.718658 21.6816) (width 0.2) (layer "F.Cu") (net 9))
 (segment (start 10.6596 19.4864) (end 7.913858 19.4864) (width 0.2) (layer "F.Cu") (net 9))
 (segment (start 1.1784 21.6816) (end 0 22.86) (width 0.2) (layer "F.Cu") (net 9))
 (segment (start 5.718658 21.6816) (end 1.1784 21.6816) (width 0.2) (layer "F.Cu") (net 9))
 (segment (start 2.67285 8.184) (end 4.695 8.184) (width 0.2) (layer "F.Cu") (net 17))
 (segment (start 0 5.51115) (end 2.67285 8.184) (width 0.2) (layer "F.Cu") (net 17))
 (segment (start 4.695 9.484) (end 3.343 9.484) (width 0.2) (layer "F.Cu") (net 18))
 (segment (start 3.343 9.484) (end 3.302 9.525) (width 0.2) (layer "F.Cu") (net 18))
 (via (at 3.302 9.525) (size 0.8) (drill 0.4) (layers "F.Cu" "B.Cu") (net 18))
 (segment (start 3.302 11.938) (end 3.302 9.525) (width 0.2) (layer "B.Cu") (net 18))
 (segment (start 0 15.24) (end 3.302 11.938) (width 0.2) (layer "B.Cu") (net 18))
 (segment (start 4.695 6.884) (end 3.472415 6.884) (width 0.2) (layer "F.Cu") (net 15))
 (segment (start 3.472415 6.884) (end 3.050604 6.462189) (width 0.2) (layer "F.Cu") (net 15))
 (via (at 3.050604 6.462189) (size 0.8) (drill 0.4) (layers "F.Cu" "B.Cu") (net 15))
 (segment (start 2.559 10.268) (end 2.559 7.06695) (width 0.2) (layer "B.Cu") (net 15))
 (segment (start 0.127 12.7) (end 2.559 10.268) (width 0.2) (layer "B.Cu") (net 15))
 (segment (start 2.559 7.06695) (end 3.050604 6.575346) (width 0.2) (layer "B.Cu") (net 15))
 (segment (start 3.050604 6.575346) (end 3.050604 6.462189) (width 0.2) (layer "B.Cu") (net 15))
 (segment (start 4.695 7.534) (end 3.0128 7.534) (width 0.2) (layer "F.Cu") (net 16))
 (segment (start 3.0128 7.534) (end 2.0574 6.5786) (width 0.2) (layer "F.Cu") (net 16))
 (via (at 2.0574 6.5786) (size 0.8) (drill 0.4) (layers "F.Cu" "B.Cu") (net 16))
 (segment (start 0 10.16) (end 2.0574 8.1026) (width 0.2) (layer "B.Cu") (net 16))
 (segment (start 2.0574 8.1026) (end 2.0574 6.5786) (width 0.2) (layer "B.Cu") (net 16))
 (segment (start 4.695 6.234) (end 5.87841 6.234) (width 0.2) (layer "F.Cu") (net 14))
 (via (at 5.87841 6.234) (size 0.8) (drill 0.4) (layers "F.Cu" "B.Cu") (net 14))
 (segment (start 0 17.78) (end 5.334 12.446) (width 0.2) (layer "B.Cu") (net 14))
 (segment (start 5.334 6.77841) (end 5.87841 6.234) (width 0.2) (layer "B.Cu") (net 14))
 (segment (start 5.334 12.446) (end 5.334 6.77841) (width 0.2) (layer "B.Cu") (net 14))
 (segment (start 14.440001 23.659999) (end 7.530999 23.659999) (width 0.2) (layer "F.Cu") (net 5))
 (segment (start 9.34585 10.134) (end 8.949556 10.530294) (width 0.2) (layer "F.Cu") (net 5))
 (segment (start 15.24 22.86) (end 14.440001 23.659999) (width 0.2) (layer "F.Cu") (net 5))
 (segment (start 6.5428 18.8364) (end 6.858 19.1516) (width 0.2) (layer "F.Cu") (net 5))
 (segment (start 4.7836 18.8364) (end 6.5428 18.8364) (width 0.2) (layer "F.Cu") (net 5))
 (segment (start 8.949556 10.530294) (end 6.886 10.530294) (width 0.2) (layer "F.Cu") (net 5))
 (segment (start 10.545 10.134) (end 9.34585 10.134) (width 0.2) (layer "F.Cu") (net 5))
 (segment (start 7.530999 23.659999) (end 7.366 23.495) (width 0.2) (layer "F.Cu") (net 5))
 (via (at 6.858 19.1516) (size 0.8) (drill 0.4) (layers "F.Cu" "B.Cu") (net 5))
 (via (at 7.366 23.495) (size 0.8) (drill 0.4) (layers "F.Cu" "B.Cu") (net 5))
 (via (at 6.886 10.530294) (size 0.8) (drill 0.4) (layers "F.Cu" "B.Cu") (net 5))
 (segment (start 7.239 23.368) (end 7.366 23.495) (width 0.2) (layer "B.Cu") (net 5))
 (segment (start 6.858 19.1516) (end 7.239 19.5326) (width 0.2) (layer "B.Cu") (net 5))
 (segment (start 7.239 19.5326) (end 7.239 23.368) (width 0.2) (layer "B.Cu") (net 5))
 (segment (start 6.731 19.0246) (end 6.731 10.685294) (width 0.2) (layer "B.Cu") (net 5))
 (segment (start 6.858 19.1516) (end 6.731 19.0246) (width 0.2) (layer "B.Cu") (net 5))
 (segment (start 6.731 10.685294) (end 6.886 10.530294) (width 0.2) (layer "B.Cu") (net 5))
 (segment (start 10.545 9.484) (end 12.024 9.484) (width 0.2) (layer "F.Cu") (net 2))
 (segment (start 8.28974 16.8864) (end 8.495914 16.680226) (width 0.2) (layer "F.Cu") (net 2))
 (segment (start 4.7836 16.8864) (end 8.28974 16.8864) (width 0.2) (layer "F.Cu") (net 2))
 (segment (start 9.0059 9.484) (end 8.788316 9.701584) (width 0.2) (layer "F.Cu") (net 2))
 (segment (start 10.545 9.484) (end 9.0059 9.484) (width 0.2) (layer "F.Cu") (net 2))
 (segment (start 12.024 9.484) (end 15.24 12.7) (width 0.2) (layer "F.Cu") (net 2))
 (via (at 8.495914 16.680226) (size 0.8) (drill 0.4) (layers "F.Cu" "B.Cu") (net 2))
 (via (at 8.788316 9.701584) (size 0.8) (drill 0.4) (layers "F.Cu" "B.Cu") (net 2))
 (segment (start 8.495914 16.680226) (end 8.927939 16.248201) (width 0.2) (layer "B.Cu") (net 2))
 (segment (start 8.927939 16.248201) (end 8.927939 9.841207) (width 0.2) (layer "B.Cu") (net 2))
 (segment (start 8.927939 9.841207) (end 8.788316 9.701584) (width 0.2) (layer "B.Cu") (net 2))
 (segment (start 12.224706 23.0632) (end 8.360396 23.0632) (width 0.2) (layer "F.Cu") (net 4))
 (segment (start 10.489 8.89) (end 7.62 8.89) (width 0.2) (layer "F.Cu") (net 4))
 (segment (start 7.380998 18.1864) (end 7.431 18.236402) (width 0.2) (layer "F.Cu") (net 4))
 (segment (start 8.360396 23.0632) (end 8.128 22.830804) (width 0.2) (layer "F.Cu") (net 4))
 (segment (start 12.929291 22.358615) (end 12.224706 23.0632) (width 0.2) (layer "F.Cu") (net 4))
 (segment (start 4.7836 18.1864) (end 7.380998 18.1864) (width 0.2) (layer "F.Cu") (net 4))
 (via (at 7.62 8.89) (size 0.8) (drill 0.4) (layers "F.Cu" "B.Cu") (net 4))
 (via (at 12.929291 22.358615) (size 0.8) (drill 0.4) (layers "F.Cu" "B.Cu") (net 4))
 (via (at 8.128 22.830804) (size 0.8) (drill 0.4) (layers "F.Cu" "B.Cu") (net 4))
 (via (at 7.431 18.236402) (size 0.8) (drill 0.4) (layers "F.Cu" "B.Cu") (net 4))
 (segment (start 7.2056 18.011002) (end 7.431 18.236402) (width 0.2) (layer "B.Cu") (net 4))
 (segment (start 13.0724 19.9476) (end 13.0724 22.215506) (width 0.2) (layer "B.Cu") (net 4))
 (segment (start 7.721544 18.526946) (end 7.721544 22.424348) (width 0.2) (layer "B.Cu") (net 4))
 (segment (start 7.62 8.89) (end 7.62 10.786244) (width 0.2) (layer "B.Cu") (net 4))
 (segment (start 15.24 17.78) (end 13.0724 19.9476) (width 0.2) (layer "B.Cu") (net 4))
 (segment (start 7.721544 22.424348) (end 8.128 22.830804) (width 0.2) (layer "B.Cu") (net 4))
 (segment (start 13.0724 22.215506) (end 12.929291 22.358615) (width 0.2) (layer "B.Cu") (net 4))
 (segment (start 7.431 18.236402) (end 7.721544 18.526946) (width 0.2) (layer "B.Cu") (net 4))
 (segment (start 7.62 10.786244) (end 7.2056 11.200644) (width 0.2) (layer "B.Cu") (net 4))
 (segment (start 7.2056 11.200644) (end 7.2056 18.011002) (width 0.2) (layer "B.Cu") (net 4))
 (segment (start 13.264 8.184) (end 10.545 8.184) (width 0.2) (layer "F.Cu") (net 1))
 (segment (start 10.545 8.184) (end 8.641992 8.184) (width 0.2) (layer "F.Cu") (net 1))
 (segment (start 8.641992 8.184) (end 8.636 8.189992) (width 0.2) (layer "F.Cu") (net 1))
 (segment (start 7.546497 16.2364) (end 7.920625 15.862272) (width 0.2) (layer "F.Cu") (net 1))
 (segment (start 15.24 10.16) (end 13.264 8.184) (width 0.2) (layer "F.Cu") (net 1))
 (segment (start 4.7836 16.2364) (end 7.546497 16.2364) (width 0.2) (layer "F.Cu") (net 1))
 (via (at 8.636 8.189992) (size 0.8) (drill 0.4) (layers "F.Cu" "B.Cu") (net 1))
 (via (at 7.920625 15.862272) (size 0.8) (drill 0.4) (layers "F.Cu" "B.Cu") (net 1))
 (segment (start 7.920625 15.862272) (end 8.02 15.762897) (width 0.2) (layer "B.Cu") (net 1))
 (segment (start 8.636 8.86395) (end 8.636 8.189992) (width 0.2) (layer "B.Cu") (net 1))
 (segment (start 8.02 15.762897) (end 8.02 9.47995) (width 0.2) (layer "B.Cu") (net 1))
 (segment (start 8.02 9.47995) (end 8.636 8.86395) (width 0.2) (layer "B.Cu") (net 1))
 (segment (start 8.850909 17.5364) (end 9.251551 17.937042) (width 0.2) (layer "F.Cu") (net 3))
 (segment (start 4.7836 17.5364) (end 8.850909 17.5364) (width 0.2) (layer "F.Cu") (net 3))
 (segment (start 10.78964 5.08) (end 10.71604 5.0064) (width 0.2) (layer "F.Cu") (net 3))
 (segment (start 15.24 5.08) (end 10.78964 5.08) (width 0.2) (layer "F.Cu") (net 3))
 (via (at 9.251551 17.937042) (size 0.8) (drill 0.4) (layers "F.Cu" "B.Cu") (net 3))
 (via (at 10.71604 5.0064) (size 0.8) (drill 0.4) (layers "F.Cu" "B.Cu") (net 3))
 (segment (start 10.613386 16.575207) (end 10.613386 5.109054) (width 0.2) (layer "B.Cu") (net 3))
 (segment (start 10.613386 5.109054) (end 10.71604 5.0064) (width 0.2) (layer "B.Cu") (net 3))
 (segment (start 9.251551 17.937042) (end 10.613386 16.575207) (width 0.2) (layer "B.Cu") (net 3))
 (segment (start 5.549468 19.4864) (end 6.234471 20.171403) (width 0.2) (layer "F.Cu") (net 6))
 (segment (start 4.7836 19.4864) (end 5.549468 19.4864) (width 0.2) (layer "F.Cu") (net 6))
 (segment (start 11.769626 22.1308) (end 7.079652 22.1308) (width 0.2) (layer "F.Cu") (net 6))
 (segment (start 12.3724 21.528026) (end 11.769626 22.1308) (width 0.2) (layer "F.Cu") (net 6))
 (segment (start 7.079652 22.1308) (end 6.477226 22.733226) (width 0.2) (layer "F.Cu") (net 6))
 (via (at 6.234471 20.171403) (size 0.8) (drill 0.4) (layers "F.Cu" "B.Cu") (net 6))
 (via (at 12.3724 21.528026) (size 0.8) (drill 0.4) (layers "F.Cu" "B.Cu") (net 6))
 (via (at 6.477226 22.733226) (size 0.8) (drill 0.4) (layers "F.Cu" "B.Cu") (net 6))
 (segment (start 6.477226 20.414158) (end 6.477226 22.733226) (width 0.2) (layer "B.Cu") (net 6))
 (segment (start 6.234471 20.171403) (end 6.477226 20.414158) (width 0.2) (layer "B.Cu") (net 6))
 (segment (start 15.24 15.424964) (end 12.3724 18.292564) (width 0.2) (layer "B.Cu") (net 6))
 (segment (start 12.3724 18.292564) (end 12.3724 21.528026) (width 0.2) (layer "B.Cu") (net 6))
 (segment (start 10.6596 20.367043) (end 10.372493 20.65415) (width 0.2) (layer "F.Cu") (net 8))
 (segment (start 10.6596 20.1364) (end 10.6596 20.367043) (width 0.2) (layer "F.Cu") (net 8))
 (via (at 10.372493 20.65415) (size 0.8) (drill 0.4) (layers "F.Cu" "B.Cu") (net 8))
 (segment (start 12.319 2.54) (end 15.24 2.54) (width 0.2) (layer "B.Cu") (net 8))
 (segment (start 10.372493 20.65415) (end 10.372493 17.433342) (width 0.2) (layer "B.Cu") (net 8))
 (segment (start 11.7856 3.0734) (end 12.319 2.54) (width 0.2) (layer "B.Cu") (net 8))
 (segment (start 11.7856 16.020235) (end 11.7856 3.0734) (width 0.2) (layer "B.Cu") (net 8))
 (segment (start 10.372493 17.433342) (end 11.7856 16.020235) (width 0.2) (layer "B.Cu") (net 8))
 (segment (start 8.471544 18.8364) (end 8.421544 18.7864) (width 0.2) (layer "F.Cu") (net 10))
 (segment (start 0 2.54) (end 6.98501 2.54) (width 0.2) (layer "F.Cu") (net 10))
 (segment (start 6.98501 2.54) (end 7.11201 2.667) (width 0.2) (layer "F.Cu") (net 10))
 (segment (start 10.6596 18.8364) (end 8.471544 18.8364) (width 0.2) (layer "F.Cu") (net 10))
 (via (at 7.11201 2.667) (size 0.8) (drill 0.4) (layers "F.Cu" "B.Cu") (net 10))
 (via (at 8.421544 18.7864) (size 0.8) (drill 0.4) (layers "F.Cu" "B.Cu") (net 10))
 (segment (start 9.8552 16.31089) (end 9.8552 4.9022) (width 0.2) (layer "B.Cu") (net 10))
 (segment (start 7.62 2.667) (end 7.11201 2.667) (width 0.2) (layer "B.Cu") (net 10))
 (segment (start 9.8552 4.9022) (end 7.62 2.667) (width 0.2) (layer "B.Cu") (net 10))
 (segment (start 8.421544 18.7864) (end 8.421544 17.744546) (width 0.2) (layer "B.Cu") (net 10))
 (segment (start 8.421544 17.744546) (end 9.8552 16.31089) (width 0.2) (layer "B.Cu") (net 10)))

